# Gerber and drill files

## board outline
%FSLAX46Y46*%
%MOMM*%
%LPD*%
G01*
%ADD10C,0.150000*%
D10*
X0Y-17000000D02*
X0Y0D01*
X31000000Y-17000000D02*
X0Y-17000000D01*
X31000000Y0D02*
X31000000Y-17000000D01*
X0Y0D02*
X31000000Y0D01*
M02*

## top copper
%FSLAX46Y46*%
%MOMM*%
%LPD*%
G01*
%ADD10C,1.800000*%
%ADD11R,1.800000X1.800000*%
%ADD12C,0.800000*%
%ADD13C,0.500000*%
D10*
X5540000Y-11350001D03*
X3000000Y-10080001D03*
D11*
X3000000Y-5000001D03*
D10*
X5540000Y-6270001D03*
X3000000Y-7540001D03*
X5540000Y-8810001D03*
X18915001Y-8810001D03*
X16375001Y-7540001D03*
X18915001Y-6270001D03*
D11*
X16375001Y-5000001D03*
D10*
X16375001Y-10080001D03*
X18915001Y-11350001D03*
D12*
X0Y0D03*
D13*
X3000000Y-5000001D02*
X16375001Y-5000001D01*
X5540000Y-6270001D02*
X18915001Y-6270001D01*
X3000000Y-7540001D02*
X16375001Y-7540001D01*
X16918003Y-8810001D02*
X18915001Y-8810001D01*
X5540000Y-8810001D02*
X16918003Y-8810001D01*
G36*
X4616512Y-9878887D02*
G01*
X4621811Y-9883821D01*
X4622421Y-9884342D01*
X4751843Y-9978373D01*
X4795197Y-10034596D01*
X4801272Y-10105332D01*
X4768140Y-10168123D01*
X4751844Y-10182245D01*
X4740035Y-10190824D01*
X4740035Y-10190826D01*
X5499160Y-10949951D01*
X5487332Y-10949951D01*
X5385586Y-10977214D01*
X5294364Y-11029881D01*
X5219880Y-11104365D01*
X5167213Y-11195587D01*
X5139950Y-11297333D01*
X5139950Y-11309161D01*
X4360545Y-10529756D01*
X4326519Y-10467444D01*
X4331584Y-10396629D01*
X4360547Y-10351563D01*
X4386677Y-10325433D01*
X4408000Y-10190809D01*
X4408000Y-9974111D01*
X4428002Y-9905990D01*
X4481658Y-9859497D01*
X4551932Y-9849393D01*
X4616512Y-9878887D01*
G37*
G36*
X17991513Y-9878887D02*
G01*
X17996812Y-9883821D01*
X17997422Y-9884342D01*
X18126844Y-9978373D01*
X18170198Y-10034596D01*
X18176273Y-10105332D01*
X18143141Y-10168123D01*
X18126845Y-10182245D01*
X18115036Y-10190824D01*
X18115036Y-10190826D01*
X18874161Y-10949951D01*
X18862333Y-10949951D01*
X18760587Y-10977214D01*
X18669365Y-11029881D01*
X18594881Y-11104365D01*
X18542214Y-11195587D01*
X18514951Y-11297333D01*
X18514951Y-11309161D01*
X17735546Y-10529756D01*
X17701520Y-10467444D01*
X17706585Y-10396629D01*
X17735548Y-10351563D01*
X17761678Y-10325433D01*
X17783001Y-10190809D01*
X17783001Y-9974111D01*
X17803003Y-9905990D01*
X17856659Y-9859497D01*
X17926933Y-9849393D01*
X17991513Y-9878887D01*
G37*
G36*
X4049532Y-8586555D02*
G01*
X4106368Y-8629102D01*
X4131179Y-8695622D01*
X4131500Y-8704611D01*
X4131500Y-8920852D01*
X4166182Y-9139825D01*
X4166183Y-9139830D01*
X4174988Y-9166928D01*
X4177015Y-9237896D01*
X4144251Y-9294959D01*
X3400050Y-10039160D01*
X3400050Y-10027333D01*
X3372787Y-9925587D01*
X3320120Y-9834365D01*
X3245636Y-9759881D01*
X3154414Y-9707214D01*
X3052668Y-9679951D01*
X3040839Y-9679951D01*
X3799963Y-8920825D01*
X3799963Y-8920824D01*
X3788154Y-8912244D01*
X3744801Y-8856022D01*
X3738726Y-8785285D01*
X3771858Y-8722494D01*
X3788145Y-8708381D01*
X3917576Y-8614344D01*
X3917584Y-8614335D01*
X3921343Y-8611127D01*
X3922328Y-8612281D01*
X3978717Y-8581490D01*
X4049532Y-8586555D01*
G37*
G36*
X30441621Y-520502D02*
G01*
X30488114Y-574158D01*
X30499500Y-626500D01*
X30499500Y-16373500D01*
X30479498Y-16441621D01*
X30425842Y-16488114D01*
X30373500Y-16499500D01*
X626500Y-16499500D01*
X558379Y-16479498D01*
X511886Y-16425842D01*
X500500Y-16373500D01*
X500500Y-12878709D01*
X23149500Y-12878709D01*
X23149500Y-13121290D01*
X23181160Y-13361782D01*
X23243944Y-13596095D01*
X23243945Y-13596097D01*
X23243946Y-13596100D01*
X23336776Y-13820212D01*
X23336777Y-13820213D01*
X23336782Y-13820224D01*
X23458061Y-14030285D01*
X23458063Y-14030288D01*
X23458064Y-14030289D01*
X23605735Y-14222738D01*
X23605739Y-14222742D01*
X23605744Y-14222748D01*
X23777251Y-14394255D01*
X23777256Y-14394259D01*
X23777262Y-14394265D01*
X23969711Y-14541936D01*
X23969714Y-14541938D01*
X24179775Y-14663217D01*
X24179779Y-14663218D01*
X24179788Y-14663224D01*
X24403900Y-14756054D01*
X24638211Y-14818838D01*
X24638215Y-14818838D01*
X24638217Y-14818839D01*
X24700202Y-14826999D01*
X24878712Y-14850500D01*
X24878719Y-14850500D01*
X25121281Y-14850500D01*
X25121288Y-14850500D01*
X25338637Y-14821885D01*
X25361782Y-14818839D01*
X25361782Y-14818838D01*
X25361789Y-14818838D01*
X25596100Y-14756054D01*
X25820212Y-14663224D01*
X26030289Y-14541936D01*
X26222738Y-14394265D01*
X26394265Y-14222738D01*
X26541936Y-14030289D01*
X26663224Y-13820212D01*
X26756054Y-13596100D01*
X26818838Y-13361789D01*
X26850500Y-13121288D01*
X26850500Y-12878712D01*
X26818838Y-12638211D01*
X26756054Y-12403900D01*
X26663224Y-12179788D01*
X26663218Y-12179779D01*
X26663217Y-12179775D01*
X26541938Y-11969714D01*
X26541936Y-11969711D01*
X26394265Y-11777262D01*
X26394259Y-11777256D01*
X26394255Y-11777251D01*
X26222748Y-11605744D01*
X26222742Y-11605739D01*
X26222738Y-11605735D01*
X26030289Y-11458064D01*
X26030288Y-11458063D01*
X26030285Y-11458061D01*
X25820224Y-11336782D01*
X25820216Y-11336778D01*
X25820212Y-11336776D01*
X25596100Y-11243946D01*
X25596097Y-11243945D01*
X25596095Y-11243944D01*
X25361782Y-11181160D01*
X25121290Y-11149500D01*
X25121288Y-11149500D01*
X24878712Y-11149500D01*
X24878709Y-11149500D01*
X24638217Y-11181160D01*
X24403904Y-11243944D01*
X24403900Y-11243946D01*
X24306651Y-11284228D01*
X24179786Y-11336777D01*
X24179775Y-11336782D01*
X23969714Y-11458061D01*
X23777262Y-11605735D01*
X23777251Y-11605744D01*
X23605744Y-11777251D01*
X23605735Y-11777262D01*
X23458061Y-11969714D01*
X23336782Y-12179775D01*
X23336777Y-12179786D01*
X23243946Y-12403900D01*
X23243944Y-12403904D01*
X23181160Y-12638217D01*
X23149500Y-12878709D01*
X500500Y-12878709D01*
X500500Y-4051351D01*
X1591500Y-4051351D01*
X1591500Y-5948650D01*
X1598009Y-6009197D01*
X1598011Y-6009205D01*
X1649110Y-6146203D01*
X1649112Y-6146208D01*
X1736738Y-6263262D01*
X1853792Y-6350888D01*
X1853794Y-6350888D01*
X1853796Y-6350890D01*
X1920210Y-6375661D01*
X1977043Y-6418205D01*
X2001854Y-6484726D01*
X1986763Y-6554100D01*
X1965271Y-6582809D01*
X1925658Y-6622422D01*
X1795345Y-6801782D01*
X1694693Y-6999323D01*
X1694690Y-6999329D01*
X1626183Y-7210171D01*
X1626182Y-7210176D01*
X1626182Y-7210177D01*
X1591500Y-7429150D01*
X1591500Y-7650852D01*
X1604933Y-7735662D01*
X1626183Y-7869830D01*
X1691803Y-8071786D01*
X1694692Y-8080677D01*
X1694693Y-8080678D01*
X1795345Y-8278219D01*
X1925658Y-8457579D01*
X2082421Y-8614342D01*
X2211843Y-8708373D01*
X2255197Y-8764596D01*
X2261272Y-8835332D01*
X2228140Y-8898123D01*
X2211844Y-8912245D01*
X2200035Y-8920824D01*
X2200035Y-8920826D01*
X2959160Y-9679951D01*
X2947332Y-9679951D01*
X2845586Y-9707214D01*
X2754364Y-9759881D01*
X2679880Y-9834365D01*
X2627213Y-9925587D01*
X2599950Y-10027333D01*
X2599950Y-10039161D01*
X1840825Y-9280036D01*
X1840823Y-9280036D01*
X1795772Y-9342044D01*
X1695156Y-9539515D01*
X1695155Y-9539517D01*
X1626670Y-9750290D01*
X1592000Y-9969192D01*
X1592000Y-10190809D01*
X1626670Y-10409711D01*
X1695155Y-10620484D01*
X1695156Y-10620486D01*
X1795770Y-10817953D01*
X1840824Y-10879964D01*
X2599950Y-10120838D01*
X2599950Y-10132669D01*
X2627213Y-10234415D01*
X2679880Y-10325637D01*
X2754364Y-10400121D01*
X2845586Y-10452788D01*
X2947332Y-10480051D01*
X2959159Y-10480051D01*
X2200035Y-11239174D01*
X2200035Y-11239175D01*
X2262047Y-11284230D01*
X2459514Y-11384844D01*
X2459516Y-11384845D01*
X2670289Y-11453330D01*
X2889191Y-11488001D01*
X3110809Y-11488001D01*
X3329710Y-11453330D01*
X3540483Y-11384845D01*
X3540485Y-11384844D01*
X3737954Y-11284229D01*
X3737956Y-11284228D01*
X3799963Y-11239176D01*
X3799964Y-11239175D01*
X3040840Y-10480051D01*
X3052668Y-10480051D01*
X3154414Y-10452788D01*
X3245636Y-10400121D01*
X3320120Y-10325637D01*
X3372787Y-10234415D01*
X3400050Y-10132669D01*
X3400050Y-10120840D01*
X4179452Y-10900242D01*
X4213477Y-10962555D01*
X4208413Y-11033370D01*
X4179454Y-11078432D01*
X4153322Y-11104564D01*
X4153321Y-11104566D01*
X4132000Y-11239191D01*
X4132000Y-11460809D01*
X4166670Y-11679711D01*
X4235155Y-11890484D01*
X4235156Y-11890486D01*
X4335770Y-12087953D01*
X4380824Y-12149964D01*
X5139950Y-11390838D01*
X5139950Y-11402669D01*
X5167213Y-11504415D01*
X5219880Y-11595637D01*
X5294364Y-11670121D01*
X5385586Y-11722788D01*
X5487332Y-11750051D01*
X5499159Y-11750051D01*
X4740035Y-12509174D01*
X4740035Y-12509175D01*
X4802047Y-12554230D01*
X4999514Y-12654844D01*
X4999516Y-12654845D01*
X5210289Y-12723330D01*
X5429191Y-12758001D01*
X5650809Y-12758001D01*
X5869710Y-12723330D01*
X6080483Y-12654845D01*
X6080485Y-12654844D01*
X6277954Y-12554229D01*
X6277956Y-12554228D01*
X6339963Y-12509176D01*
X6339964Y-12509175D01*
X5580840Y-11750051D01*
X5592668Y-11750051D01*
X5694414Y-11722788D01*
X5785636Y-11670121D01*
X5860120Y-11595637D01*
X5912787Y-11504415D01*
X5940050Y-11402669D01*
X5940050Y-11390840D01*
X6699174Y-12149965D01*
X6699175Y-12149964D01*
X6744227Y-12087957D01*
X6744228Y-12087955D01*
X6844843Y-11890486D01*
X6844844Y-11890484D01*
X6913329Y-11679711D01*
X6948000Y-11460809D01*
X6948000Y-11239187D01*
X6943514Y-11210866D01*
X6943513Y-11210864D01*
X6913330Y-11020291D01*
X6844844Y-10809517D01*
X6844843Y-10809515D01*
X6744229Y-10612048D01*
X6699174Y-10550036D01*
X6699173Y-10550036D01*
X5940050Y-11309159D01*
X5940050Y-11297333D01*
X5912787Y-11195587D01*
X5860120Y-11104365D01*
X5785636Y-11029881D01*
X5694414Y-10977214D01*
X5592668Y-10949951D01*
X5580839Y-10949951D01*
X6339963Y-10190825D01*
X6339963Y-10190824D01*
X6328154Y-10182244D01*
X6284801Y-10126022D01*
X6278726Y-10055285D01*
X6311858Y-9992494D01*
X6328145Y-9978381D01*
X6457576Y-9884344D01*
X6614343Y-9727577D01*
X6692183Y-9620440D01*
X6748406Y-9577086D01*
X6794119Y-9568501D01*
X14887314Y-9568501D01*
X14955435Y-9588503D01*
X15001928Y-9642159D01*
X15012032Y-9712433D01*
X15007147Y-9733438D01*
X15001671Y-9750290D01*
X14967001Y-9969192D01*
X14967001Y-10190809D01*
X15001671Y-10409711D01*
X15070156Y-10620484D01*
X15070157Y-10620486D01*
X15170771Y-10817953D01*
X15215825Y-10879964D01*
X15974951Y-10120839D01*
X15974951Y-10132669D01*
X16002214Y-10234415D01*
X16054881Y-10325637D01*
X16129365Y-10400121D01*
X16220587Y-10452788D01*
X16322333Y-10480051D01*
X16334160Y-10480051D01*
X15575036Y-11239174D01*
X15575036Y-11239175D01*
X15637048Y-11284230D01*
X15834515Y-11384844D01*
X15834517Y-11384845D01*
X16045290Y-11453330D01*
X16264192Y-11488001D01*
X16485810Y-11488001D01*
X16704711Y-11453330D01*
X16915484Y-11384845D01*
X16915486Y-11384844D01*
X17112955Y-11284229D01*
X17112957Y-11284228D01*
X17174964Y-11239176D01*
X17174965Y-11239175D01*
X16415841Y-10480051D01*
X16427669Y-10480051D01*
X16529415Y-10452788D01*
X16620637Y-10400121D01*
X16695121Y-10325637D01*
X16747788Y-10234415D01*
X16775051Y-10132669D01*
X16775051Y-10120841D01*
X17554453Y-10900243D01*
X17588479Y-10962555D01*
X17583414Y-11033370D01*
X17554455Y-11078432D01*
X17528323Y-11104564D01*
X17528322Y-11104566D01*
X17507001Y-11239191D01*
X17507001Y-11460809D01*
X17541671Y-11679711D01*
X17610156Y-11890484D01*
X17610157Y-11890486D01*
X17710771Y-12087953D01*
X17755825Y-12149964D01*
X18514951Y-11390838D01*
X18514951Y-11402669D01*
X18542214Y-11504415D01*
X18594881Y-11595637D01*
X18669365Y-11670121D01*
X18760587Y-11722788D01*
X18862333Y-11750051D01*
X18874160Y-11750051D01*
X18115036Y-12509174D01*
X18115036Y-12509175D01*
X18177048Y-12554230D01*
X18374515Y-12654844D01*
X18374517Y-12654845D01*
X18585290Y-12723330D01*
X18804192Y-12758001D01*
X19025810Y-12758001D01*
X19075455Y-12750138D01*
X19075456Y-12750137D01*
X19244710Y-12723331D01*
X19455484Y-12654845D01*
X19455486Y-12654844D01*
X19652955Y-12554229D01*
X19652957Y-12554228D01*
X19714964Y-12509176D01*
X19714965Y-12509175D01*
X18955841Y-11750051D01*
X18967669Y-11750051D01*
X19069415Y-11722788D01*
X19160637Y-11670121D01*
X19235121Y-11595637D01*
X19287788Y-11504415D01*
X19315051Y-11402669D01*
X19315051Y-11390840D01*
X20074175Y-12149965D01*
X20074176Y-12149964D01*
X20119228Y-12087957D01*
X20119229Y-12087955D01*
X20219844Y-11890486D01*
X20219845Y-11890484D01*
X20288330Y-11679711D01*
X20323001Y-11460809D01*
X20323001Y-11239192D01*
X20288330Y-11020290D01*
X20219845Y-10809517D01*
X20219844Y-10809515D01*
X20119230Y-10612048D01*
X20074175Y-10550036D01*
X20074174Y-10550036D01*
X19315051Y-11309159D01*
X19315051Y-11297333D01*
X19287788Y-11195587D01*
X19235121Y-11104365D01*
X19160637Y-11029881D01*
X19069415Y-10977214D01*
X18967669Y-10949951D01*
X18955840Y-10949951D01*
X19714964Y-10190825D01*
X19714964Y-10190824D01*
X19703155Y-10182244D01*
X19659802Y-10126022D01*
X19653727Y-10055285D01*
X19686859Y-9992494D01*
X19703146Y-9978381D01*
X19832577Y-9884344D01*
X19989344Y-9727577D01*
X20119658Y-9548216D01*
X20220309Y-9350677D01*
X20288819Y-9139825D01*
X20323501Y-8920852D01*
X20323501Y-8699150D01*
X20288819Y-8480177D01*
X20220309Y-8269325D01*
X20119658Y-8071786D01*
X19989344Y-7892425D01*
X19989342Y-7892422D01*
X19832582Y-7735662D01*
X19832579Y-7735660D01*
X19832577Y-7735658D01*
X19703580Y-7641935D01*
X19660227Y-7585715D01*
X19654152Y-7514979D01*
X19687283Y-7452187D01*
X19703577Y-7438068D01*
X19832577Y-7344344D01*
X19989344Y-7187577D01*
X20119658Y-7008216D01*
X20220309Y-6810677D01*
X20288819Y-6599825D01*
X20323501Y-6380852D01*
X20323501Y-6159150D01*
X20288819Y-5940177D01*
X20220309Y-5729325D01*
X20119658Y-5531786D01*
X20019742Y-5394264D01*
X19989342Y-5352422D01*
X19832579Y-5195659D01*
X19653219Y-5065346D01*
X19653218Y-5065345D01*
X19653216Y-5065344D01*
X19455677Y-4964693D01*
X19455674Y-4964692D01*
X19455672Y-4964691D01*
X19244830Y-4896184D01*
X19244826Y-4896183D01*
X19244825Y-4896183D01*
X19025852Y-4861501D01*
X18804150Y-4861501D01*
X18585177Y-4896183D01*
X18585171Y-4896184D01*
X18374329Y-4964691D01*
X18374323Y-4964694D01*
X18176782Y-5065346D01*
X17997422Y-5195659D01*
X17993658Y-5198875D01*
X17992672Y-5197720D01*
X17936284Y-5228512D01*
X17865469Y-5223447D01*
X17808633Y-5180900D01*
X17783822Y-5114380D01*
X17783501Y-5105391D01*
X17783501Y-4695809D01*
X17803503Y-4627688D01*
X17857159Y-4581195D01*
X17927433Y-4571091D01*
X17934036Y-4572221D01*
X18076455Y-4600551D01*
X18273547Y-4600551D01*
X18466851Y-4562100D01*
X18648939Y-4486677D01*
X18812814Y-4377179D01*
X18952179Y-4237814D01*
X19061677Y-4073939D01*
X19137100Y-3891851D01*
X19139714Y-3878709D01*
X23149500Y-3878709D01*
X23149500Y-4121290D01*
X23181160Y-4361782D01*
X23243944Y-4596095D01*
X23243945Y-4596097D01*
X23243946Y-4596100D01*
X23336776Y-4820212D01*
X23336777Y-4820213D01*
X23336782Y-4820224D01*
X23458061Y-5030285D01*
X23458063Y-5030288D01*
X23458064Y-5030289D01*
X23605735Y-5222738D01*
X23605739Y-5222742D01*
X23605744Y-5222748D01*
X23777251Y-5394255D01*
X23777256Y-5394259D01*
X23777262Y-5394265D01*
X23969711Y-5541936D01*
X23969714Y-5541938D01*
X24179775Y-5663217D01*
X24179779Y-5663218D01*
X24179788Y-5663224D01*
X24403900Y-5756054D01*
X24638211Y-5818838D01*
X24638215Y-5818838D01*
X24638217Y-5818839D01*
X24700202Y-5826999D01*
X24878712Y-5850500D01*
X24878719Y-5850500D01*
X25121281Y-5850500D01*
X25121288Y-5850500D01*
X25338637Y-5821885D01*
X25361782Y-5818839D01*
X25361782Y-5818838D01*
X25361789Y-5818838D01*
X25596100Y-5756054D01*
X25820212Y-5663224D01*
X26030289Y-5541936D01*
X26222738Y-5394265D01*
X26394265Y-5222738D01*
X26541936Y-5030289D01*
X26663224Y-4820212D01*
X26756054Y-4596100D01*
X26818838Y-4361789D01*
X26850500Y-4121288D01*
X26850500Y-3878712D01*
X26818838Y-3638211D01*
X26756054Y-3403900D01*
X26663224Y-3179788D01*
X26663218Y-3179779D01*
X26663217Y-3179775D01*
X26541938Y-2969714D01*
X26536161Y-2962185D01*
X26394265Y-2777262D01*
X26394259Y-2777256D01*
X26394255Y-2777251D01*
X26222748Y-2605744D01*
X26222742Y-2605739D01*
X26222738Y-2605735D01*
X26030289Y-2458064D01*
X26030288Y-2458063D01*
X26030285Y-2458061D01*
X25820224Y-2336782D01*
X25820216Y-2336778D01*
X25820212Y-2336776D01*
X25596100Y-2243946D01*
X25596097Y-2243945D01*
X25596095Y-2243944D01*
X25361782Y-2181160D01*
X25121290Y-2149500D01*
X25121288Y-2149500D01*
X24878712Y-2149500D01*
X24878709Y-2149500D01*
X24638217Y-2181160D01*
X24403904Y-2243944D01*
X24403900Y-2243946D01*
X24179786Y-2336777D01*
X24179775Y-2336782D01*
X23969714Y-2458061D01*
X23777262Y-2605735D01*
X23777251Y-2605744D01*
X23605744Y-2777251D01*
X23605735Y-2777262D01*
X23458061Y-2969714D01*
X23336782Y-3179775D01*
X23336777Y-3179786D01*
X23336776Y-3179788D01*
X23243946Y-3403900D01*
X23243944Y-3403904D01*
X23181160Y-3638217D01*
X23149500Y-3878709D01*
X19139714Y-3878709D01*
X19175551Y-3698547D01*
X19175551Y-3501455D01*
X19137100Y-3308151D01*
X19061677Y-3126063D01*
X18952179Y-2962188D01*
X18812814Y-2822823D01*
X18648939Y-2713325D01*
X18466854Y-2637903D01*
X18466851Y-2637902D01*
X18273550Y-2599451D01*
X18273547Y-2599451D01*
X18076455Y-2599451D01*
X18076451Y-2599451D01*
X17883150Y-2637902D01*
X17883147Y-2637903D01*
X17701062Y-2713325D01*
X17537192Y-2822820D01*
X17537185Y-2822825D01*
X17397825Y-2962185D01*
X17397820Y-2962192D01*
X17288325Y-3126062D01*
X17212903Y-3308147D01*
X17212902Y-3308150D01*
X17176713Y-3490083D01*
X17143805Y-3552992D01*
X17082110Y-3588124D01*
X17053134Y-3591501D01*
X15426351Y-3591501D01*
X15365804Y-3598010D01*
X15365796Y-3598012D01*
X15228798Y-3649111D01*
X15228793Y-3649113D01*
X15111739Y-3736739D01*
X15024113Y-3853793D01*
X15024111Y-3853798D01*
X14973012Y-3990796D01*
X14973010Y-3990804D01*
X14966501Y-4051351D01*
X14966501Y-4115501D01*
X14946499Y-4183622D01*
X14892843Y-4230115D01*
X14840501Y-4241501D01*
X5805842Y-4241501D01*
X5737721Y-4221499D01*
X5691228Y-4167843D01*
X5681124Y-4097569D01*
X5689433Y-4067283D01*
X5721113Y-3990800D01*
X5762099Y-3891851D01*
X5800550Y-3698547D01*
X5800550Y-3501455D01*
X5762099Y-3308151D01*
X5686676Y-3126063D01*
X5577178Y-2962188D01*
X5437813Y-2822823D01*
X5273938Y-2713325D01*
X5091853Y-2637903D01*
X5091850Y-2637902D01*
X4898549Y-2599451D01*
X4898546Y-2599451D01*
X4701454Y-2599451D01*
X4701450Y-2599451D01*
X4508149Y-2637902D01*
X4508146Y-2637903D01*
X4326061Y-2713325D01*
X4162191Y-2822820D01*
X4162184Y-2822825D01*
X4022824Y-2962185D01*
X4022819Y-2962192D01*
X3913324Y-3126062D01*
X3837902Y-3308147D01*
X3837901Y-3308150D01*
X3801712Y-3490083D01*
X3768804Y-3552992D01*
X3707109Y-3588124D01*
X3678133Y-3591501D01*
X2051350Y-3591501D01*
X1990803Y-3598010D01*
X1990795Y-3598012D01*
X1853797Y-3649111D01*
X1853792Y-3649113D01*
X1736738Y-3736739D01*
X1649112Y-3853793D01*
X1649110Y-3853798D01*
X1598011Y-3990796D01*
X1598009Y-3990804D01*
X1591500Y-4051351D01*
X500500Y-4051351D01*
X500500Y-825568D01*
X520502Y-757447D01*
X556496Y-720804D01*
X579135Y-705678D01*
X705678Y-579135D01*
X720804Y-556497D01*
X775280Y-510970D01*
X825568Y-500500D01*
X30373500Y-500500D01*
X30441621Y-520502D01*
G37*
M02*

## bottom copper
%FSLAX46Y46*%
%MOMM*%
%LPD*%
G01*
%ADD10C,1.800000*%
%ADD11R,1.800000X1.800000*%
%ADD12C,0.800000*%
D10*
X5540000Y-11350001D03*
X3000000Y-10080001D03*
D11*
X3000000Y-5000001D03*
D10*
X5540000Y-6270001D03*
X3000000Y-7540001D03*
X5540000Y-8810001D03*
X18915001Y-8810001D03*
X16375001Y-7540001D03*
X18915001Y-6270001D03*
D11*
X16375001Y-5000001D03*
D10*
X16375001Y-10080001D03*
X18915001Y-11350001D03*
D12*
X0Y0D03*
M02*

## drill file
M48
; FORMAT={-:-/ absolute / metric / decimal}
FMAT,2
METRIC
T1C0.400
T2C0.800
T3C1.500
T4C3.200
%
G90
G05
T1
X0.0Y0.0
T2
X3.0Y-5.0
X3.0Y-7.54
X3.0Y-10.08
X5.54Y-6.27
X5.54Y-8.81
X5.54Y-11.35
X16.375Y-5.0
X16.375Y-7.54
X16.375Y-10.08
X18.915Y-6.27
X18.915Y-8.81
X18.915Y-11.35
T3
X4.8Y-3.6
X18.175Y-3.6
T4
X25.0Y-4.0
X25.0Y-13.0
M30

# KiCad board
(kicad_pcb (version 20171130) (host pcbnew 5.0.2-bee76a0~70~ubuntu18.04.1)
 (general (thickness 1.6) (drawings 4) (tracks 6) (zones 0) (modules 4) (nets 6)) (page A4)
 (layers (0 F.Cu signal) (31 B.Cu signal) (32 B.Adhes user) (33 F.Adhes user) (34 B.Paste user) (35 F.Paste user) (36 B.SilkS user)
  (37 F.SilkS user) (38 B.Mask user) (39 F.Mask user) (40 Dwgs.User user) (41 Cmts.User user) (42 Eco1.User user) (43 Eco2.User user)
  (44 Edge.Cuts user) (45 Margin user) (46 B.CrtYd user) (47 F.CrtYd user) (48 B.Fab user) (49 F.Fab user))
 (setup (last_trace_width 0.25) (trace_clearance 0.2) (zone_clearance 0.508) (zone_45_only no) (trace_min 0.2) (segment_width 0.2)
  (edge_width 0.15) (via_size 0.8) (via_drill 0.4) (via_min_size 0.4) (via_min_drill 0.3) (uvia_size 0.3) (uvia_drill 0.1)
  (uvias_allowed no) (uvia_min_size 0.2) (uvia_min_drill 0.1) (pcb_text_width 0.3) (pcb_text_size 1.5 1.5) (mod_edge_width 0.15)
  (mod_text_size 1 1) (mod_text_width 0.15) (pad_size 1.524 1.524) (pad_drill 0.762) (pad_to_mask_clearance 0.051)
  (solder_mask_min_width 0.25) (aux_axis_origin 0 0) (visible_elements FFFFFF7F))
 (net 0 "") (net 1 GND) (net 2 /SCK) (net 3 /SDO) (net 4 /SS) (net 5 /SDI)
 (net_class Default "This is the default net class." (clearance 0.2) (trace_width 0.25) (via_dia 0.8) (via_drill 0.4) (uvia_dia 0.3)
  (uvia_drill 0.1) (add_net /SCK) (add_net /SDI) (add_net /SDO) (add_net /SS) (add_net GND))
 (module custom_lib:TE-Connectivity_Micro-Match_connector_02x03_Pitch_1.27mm (layer F.Cu) (at 3 5.000001)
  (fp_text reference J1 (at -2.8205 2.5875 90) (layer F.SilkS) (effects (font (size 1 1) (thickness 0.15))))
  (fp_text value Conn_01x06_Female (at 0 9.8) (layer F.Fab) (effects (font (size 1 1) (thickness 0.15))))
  (pad 6 thru_hole circle (at 2.54 6.35) (size 1.8 1.8) (drill 0.8001) (layers *.Cu *.Mask) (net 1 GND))
  (pad 5 thru_hole circle (at 0 5.08) (size 1.8 1.8) (drill 0.8001) (layers *.Cu *.Mask) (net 1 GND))
  (pad 1 thru_hole rect (at 0 0) (size 1.8 1.8) (drill 0.8001) (layers *.Cu *.Mask) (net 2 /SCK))
  (pad 2 thru_hole circle (at 2.54 1.27) (size 1.8 1.8) (drill 0.8001) (layers *.Cu *.Mask) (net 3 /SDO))
  (pad 3 thru_hole circle (at 0 2.54) (size 1.8 1.8) (drill 0.8001) (layers *.Cu *.Mask) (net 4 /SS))
  (pad 4 thru_hole circle (at 2.54 3.81) (size 1.8 1.8) (drill 0.8001) (layers *.Cu *.Mask) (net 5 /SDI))
  (pad "" np_thru_hole circle (at 1.8 -1.4) (size 1.5001 1.5001) (drill 1.5001) (layers *.Cu *.Mask)))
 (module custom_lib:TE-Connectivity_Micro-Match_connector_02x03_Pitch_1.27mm (layer F.Cu) (at 16.375001 5.000001)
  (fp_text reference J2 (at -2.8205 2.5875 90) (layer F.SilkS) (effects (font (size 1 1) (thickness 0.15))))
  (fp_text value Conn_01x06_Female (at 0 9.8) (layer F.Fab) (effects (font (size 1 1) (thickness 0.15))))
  (pad "" np_thru_hole circle (at 1.8 -1.4) (size 1.5001 1.5001) (drill 1.5001) (layers *.Cu *.Mask))
  (pad 4 thru_hole circle (at 2.54 3.81) (size 1.8 1.8) (drill 0.8001) (layers *.Cu *.Mask) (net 5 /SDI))
  (pad 3 thru_hole circle (at 0 2.54) (size 1.8 1.8) (drill 0.8001) (layers *.Cu *.Mask) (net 4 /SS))
  (pad 2 thru_hole circle (at 2.54 1.27) (size 1.8 1.8) (drill 0.8001) (layers *.Cu *.Mask) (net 3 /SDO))
  (pad 1 thru_hole rect (at 0 0) (size 1.8 1.8) (drill 0.8001) (layers *.Cu *.Mask) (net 2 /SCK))
  (pad 5 thru_hole circle (at 0 5.08) (size 1.8 1.8) (drill 0.8001) (layers *.Cu *.Mask) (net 1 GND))
  (pad 6 thru_hole circle (at 2.54 6.35) (size 1.8 1.8) (drill 0.8001) (layers *.Cu *.Mask) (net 1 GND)))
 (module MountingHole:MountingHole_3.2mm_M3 (layer F.Cu) (at 25 4)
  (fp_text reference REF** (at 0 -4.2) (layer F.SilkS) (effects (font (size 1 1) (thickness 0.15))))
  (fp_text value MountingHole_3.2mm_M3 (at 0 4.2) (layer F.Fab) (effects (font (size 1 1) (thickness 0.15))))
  (pad 1 np_thru_hole circle (at 0 0) (size 3.2 3.2) (drill 3.2) (layers *.Cu *.Mask)))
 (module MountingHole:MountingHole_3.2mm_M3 (layer F.Cu) (at 25 13)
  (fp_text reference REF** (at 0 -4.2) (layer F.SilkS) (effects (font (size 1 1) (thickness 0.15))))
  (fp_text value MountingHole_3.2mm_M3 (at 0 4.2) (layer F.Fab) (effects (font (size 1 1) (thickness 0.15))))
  (pad 1 np_thru_hole circle (at 0 0) (size 3.2 3.2) (drill 3.2) (layers *.Cu *.Mask)))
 (gr_line (start 0 17) (end 0 0) (layer Edge.Cuts) (width 0.15))
 (gr_line (start 31 17) (end 0 17) (layer Edge.Cuts) (width 0.15))
 (gr_line (start 31 0) (end 31 17) (layer Edge.Cuts) (width 0.15))
 (gr_line (start 0 0) (end 31 0) (layer Edge.Cuts) (width 0.15))
 (via (at 0 0) (size 0.8) (drill 0.4) (layers F.Cu B.Cu) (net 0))
 (segment (start 3 5.000001) (end 16.375001 5.000001) (width 0.5) (layer F.Cu) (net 2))
 (segment (start 5.54 6.270001) (end 18.915001 6.270001) (width 0.5) (layer F.Cu) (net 3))
 (segment (start 3 7.540001) (end 16.375001 7.540001) (width 0.5) (layer F.Cu) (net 4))
 (segment (start 16.918003 8.810001) (end 18.915001 8.810001) (width 0.5) (layer F.Cu) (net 5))
 (segment (start 5.54 8.810001) (end 16.918003 8.810001) (width 0.5) (layer F.Cu) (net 5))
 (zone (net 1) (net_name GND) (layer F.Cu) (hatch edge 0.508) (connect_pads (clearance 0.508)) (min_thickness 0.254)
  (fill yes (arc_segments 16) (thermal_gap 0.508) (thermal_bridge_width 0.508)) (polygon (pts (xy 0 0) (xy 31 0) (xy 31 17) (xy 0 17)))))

